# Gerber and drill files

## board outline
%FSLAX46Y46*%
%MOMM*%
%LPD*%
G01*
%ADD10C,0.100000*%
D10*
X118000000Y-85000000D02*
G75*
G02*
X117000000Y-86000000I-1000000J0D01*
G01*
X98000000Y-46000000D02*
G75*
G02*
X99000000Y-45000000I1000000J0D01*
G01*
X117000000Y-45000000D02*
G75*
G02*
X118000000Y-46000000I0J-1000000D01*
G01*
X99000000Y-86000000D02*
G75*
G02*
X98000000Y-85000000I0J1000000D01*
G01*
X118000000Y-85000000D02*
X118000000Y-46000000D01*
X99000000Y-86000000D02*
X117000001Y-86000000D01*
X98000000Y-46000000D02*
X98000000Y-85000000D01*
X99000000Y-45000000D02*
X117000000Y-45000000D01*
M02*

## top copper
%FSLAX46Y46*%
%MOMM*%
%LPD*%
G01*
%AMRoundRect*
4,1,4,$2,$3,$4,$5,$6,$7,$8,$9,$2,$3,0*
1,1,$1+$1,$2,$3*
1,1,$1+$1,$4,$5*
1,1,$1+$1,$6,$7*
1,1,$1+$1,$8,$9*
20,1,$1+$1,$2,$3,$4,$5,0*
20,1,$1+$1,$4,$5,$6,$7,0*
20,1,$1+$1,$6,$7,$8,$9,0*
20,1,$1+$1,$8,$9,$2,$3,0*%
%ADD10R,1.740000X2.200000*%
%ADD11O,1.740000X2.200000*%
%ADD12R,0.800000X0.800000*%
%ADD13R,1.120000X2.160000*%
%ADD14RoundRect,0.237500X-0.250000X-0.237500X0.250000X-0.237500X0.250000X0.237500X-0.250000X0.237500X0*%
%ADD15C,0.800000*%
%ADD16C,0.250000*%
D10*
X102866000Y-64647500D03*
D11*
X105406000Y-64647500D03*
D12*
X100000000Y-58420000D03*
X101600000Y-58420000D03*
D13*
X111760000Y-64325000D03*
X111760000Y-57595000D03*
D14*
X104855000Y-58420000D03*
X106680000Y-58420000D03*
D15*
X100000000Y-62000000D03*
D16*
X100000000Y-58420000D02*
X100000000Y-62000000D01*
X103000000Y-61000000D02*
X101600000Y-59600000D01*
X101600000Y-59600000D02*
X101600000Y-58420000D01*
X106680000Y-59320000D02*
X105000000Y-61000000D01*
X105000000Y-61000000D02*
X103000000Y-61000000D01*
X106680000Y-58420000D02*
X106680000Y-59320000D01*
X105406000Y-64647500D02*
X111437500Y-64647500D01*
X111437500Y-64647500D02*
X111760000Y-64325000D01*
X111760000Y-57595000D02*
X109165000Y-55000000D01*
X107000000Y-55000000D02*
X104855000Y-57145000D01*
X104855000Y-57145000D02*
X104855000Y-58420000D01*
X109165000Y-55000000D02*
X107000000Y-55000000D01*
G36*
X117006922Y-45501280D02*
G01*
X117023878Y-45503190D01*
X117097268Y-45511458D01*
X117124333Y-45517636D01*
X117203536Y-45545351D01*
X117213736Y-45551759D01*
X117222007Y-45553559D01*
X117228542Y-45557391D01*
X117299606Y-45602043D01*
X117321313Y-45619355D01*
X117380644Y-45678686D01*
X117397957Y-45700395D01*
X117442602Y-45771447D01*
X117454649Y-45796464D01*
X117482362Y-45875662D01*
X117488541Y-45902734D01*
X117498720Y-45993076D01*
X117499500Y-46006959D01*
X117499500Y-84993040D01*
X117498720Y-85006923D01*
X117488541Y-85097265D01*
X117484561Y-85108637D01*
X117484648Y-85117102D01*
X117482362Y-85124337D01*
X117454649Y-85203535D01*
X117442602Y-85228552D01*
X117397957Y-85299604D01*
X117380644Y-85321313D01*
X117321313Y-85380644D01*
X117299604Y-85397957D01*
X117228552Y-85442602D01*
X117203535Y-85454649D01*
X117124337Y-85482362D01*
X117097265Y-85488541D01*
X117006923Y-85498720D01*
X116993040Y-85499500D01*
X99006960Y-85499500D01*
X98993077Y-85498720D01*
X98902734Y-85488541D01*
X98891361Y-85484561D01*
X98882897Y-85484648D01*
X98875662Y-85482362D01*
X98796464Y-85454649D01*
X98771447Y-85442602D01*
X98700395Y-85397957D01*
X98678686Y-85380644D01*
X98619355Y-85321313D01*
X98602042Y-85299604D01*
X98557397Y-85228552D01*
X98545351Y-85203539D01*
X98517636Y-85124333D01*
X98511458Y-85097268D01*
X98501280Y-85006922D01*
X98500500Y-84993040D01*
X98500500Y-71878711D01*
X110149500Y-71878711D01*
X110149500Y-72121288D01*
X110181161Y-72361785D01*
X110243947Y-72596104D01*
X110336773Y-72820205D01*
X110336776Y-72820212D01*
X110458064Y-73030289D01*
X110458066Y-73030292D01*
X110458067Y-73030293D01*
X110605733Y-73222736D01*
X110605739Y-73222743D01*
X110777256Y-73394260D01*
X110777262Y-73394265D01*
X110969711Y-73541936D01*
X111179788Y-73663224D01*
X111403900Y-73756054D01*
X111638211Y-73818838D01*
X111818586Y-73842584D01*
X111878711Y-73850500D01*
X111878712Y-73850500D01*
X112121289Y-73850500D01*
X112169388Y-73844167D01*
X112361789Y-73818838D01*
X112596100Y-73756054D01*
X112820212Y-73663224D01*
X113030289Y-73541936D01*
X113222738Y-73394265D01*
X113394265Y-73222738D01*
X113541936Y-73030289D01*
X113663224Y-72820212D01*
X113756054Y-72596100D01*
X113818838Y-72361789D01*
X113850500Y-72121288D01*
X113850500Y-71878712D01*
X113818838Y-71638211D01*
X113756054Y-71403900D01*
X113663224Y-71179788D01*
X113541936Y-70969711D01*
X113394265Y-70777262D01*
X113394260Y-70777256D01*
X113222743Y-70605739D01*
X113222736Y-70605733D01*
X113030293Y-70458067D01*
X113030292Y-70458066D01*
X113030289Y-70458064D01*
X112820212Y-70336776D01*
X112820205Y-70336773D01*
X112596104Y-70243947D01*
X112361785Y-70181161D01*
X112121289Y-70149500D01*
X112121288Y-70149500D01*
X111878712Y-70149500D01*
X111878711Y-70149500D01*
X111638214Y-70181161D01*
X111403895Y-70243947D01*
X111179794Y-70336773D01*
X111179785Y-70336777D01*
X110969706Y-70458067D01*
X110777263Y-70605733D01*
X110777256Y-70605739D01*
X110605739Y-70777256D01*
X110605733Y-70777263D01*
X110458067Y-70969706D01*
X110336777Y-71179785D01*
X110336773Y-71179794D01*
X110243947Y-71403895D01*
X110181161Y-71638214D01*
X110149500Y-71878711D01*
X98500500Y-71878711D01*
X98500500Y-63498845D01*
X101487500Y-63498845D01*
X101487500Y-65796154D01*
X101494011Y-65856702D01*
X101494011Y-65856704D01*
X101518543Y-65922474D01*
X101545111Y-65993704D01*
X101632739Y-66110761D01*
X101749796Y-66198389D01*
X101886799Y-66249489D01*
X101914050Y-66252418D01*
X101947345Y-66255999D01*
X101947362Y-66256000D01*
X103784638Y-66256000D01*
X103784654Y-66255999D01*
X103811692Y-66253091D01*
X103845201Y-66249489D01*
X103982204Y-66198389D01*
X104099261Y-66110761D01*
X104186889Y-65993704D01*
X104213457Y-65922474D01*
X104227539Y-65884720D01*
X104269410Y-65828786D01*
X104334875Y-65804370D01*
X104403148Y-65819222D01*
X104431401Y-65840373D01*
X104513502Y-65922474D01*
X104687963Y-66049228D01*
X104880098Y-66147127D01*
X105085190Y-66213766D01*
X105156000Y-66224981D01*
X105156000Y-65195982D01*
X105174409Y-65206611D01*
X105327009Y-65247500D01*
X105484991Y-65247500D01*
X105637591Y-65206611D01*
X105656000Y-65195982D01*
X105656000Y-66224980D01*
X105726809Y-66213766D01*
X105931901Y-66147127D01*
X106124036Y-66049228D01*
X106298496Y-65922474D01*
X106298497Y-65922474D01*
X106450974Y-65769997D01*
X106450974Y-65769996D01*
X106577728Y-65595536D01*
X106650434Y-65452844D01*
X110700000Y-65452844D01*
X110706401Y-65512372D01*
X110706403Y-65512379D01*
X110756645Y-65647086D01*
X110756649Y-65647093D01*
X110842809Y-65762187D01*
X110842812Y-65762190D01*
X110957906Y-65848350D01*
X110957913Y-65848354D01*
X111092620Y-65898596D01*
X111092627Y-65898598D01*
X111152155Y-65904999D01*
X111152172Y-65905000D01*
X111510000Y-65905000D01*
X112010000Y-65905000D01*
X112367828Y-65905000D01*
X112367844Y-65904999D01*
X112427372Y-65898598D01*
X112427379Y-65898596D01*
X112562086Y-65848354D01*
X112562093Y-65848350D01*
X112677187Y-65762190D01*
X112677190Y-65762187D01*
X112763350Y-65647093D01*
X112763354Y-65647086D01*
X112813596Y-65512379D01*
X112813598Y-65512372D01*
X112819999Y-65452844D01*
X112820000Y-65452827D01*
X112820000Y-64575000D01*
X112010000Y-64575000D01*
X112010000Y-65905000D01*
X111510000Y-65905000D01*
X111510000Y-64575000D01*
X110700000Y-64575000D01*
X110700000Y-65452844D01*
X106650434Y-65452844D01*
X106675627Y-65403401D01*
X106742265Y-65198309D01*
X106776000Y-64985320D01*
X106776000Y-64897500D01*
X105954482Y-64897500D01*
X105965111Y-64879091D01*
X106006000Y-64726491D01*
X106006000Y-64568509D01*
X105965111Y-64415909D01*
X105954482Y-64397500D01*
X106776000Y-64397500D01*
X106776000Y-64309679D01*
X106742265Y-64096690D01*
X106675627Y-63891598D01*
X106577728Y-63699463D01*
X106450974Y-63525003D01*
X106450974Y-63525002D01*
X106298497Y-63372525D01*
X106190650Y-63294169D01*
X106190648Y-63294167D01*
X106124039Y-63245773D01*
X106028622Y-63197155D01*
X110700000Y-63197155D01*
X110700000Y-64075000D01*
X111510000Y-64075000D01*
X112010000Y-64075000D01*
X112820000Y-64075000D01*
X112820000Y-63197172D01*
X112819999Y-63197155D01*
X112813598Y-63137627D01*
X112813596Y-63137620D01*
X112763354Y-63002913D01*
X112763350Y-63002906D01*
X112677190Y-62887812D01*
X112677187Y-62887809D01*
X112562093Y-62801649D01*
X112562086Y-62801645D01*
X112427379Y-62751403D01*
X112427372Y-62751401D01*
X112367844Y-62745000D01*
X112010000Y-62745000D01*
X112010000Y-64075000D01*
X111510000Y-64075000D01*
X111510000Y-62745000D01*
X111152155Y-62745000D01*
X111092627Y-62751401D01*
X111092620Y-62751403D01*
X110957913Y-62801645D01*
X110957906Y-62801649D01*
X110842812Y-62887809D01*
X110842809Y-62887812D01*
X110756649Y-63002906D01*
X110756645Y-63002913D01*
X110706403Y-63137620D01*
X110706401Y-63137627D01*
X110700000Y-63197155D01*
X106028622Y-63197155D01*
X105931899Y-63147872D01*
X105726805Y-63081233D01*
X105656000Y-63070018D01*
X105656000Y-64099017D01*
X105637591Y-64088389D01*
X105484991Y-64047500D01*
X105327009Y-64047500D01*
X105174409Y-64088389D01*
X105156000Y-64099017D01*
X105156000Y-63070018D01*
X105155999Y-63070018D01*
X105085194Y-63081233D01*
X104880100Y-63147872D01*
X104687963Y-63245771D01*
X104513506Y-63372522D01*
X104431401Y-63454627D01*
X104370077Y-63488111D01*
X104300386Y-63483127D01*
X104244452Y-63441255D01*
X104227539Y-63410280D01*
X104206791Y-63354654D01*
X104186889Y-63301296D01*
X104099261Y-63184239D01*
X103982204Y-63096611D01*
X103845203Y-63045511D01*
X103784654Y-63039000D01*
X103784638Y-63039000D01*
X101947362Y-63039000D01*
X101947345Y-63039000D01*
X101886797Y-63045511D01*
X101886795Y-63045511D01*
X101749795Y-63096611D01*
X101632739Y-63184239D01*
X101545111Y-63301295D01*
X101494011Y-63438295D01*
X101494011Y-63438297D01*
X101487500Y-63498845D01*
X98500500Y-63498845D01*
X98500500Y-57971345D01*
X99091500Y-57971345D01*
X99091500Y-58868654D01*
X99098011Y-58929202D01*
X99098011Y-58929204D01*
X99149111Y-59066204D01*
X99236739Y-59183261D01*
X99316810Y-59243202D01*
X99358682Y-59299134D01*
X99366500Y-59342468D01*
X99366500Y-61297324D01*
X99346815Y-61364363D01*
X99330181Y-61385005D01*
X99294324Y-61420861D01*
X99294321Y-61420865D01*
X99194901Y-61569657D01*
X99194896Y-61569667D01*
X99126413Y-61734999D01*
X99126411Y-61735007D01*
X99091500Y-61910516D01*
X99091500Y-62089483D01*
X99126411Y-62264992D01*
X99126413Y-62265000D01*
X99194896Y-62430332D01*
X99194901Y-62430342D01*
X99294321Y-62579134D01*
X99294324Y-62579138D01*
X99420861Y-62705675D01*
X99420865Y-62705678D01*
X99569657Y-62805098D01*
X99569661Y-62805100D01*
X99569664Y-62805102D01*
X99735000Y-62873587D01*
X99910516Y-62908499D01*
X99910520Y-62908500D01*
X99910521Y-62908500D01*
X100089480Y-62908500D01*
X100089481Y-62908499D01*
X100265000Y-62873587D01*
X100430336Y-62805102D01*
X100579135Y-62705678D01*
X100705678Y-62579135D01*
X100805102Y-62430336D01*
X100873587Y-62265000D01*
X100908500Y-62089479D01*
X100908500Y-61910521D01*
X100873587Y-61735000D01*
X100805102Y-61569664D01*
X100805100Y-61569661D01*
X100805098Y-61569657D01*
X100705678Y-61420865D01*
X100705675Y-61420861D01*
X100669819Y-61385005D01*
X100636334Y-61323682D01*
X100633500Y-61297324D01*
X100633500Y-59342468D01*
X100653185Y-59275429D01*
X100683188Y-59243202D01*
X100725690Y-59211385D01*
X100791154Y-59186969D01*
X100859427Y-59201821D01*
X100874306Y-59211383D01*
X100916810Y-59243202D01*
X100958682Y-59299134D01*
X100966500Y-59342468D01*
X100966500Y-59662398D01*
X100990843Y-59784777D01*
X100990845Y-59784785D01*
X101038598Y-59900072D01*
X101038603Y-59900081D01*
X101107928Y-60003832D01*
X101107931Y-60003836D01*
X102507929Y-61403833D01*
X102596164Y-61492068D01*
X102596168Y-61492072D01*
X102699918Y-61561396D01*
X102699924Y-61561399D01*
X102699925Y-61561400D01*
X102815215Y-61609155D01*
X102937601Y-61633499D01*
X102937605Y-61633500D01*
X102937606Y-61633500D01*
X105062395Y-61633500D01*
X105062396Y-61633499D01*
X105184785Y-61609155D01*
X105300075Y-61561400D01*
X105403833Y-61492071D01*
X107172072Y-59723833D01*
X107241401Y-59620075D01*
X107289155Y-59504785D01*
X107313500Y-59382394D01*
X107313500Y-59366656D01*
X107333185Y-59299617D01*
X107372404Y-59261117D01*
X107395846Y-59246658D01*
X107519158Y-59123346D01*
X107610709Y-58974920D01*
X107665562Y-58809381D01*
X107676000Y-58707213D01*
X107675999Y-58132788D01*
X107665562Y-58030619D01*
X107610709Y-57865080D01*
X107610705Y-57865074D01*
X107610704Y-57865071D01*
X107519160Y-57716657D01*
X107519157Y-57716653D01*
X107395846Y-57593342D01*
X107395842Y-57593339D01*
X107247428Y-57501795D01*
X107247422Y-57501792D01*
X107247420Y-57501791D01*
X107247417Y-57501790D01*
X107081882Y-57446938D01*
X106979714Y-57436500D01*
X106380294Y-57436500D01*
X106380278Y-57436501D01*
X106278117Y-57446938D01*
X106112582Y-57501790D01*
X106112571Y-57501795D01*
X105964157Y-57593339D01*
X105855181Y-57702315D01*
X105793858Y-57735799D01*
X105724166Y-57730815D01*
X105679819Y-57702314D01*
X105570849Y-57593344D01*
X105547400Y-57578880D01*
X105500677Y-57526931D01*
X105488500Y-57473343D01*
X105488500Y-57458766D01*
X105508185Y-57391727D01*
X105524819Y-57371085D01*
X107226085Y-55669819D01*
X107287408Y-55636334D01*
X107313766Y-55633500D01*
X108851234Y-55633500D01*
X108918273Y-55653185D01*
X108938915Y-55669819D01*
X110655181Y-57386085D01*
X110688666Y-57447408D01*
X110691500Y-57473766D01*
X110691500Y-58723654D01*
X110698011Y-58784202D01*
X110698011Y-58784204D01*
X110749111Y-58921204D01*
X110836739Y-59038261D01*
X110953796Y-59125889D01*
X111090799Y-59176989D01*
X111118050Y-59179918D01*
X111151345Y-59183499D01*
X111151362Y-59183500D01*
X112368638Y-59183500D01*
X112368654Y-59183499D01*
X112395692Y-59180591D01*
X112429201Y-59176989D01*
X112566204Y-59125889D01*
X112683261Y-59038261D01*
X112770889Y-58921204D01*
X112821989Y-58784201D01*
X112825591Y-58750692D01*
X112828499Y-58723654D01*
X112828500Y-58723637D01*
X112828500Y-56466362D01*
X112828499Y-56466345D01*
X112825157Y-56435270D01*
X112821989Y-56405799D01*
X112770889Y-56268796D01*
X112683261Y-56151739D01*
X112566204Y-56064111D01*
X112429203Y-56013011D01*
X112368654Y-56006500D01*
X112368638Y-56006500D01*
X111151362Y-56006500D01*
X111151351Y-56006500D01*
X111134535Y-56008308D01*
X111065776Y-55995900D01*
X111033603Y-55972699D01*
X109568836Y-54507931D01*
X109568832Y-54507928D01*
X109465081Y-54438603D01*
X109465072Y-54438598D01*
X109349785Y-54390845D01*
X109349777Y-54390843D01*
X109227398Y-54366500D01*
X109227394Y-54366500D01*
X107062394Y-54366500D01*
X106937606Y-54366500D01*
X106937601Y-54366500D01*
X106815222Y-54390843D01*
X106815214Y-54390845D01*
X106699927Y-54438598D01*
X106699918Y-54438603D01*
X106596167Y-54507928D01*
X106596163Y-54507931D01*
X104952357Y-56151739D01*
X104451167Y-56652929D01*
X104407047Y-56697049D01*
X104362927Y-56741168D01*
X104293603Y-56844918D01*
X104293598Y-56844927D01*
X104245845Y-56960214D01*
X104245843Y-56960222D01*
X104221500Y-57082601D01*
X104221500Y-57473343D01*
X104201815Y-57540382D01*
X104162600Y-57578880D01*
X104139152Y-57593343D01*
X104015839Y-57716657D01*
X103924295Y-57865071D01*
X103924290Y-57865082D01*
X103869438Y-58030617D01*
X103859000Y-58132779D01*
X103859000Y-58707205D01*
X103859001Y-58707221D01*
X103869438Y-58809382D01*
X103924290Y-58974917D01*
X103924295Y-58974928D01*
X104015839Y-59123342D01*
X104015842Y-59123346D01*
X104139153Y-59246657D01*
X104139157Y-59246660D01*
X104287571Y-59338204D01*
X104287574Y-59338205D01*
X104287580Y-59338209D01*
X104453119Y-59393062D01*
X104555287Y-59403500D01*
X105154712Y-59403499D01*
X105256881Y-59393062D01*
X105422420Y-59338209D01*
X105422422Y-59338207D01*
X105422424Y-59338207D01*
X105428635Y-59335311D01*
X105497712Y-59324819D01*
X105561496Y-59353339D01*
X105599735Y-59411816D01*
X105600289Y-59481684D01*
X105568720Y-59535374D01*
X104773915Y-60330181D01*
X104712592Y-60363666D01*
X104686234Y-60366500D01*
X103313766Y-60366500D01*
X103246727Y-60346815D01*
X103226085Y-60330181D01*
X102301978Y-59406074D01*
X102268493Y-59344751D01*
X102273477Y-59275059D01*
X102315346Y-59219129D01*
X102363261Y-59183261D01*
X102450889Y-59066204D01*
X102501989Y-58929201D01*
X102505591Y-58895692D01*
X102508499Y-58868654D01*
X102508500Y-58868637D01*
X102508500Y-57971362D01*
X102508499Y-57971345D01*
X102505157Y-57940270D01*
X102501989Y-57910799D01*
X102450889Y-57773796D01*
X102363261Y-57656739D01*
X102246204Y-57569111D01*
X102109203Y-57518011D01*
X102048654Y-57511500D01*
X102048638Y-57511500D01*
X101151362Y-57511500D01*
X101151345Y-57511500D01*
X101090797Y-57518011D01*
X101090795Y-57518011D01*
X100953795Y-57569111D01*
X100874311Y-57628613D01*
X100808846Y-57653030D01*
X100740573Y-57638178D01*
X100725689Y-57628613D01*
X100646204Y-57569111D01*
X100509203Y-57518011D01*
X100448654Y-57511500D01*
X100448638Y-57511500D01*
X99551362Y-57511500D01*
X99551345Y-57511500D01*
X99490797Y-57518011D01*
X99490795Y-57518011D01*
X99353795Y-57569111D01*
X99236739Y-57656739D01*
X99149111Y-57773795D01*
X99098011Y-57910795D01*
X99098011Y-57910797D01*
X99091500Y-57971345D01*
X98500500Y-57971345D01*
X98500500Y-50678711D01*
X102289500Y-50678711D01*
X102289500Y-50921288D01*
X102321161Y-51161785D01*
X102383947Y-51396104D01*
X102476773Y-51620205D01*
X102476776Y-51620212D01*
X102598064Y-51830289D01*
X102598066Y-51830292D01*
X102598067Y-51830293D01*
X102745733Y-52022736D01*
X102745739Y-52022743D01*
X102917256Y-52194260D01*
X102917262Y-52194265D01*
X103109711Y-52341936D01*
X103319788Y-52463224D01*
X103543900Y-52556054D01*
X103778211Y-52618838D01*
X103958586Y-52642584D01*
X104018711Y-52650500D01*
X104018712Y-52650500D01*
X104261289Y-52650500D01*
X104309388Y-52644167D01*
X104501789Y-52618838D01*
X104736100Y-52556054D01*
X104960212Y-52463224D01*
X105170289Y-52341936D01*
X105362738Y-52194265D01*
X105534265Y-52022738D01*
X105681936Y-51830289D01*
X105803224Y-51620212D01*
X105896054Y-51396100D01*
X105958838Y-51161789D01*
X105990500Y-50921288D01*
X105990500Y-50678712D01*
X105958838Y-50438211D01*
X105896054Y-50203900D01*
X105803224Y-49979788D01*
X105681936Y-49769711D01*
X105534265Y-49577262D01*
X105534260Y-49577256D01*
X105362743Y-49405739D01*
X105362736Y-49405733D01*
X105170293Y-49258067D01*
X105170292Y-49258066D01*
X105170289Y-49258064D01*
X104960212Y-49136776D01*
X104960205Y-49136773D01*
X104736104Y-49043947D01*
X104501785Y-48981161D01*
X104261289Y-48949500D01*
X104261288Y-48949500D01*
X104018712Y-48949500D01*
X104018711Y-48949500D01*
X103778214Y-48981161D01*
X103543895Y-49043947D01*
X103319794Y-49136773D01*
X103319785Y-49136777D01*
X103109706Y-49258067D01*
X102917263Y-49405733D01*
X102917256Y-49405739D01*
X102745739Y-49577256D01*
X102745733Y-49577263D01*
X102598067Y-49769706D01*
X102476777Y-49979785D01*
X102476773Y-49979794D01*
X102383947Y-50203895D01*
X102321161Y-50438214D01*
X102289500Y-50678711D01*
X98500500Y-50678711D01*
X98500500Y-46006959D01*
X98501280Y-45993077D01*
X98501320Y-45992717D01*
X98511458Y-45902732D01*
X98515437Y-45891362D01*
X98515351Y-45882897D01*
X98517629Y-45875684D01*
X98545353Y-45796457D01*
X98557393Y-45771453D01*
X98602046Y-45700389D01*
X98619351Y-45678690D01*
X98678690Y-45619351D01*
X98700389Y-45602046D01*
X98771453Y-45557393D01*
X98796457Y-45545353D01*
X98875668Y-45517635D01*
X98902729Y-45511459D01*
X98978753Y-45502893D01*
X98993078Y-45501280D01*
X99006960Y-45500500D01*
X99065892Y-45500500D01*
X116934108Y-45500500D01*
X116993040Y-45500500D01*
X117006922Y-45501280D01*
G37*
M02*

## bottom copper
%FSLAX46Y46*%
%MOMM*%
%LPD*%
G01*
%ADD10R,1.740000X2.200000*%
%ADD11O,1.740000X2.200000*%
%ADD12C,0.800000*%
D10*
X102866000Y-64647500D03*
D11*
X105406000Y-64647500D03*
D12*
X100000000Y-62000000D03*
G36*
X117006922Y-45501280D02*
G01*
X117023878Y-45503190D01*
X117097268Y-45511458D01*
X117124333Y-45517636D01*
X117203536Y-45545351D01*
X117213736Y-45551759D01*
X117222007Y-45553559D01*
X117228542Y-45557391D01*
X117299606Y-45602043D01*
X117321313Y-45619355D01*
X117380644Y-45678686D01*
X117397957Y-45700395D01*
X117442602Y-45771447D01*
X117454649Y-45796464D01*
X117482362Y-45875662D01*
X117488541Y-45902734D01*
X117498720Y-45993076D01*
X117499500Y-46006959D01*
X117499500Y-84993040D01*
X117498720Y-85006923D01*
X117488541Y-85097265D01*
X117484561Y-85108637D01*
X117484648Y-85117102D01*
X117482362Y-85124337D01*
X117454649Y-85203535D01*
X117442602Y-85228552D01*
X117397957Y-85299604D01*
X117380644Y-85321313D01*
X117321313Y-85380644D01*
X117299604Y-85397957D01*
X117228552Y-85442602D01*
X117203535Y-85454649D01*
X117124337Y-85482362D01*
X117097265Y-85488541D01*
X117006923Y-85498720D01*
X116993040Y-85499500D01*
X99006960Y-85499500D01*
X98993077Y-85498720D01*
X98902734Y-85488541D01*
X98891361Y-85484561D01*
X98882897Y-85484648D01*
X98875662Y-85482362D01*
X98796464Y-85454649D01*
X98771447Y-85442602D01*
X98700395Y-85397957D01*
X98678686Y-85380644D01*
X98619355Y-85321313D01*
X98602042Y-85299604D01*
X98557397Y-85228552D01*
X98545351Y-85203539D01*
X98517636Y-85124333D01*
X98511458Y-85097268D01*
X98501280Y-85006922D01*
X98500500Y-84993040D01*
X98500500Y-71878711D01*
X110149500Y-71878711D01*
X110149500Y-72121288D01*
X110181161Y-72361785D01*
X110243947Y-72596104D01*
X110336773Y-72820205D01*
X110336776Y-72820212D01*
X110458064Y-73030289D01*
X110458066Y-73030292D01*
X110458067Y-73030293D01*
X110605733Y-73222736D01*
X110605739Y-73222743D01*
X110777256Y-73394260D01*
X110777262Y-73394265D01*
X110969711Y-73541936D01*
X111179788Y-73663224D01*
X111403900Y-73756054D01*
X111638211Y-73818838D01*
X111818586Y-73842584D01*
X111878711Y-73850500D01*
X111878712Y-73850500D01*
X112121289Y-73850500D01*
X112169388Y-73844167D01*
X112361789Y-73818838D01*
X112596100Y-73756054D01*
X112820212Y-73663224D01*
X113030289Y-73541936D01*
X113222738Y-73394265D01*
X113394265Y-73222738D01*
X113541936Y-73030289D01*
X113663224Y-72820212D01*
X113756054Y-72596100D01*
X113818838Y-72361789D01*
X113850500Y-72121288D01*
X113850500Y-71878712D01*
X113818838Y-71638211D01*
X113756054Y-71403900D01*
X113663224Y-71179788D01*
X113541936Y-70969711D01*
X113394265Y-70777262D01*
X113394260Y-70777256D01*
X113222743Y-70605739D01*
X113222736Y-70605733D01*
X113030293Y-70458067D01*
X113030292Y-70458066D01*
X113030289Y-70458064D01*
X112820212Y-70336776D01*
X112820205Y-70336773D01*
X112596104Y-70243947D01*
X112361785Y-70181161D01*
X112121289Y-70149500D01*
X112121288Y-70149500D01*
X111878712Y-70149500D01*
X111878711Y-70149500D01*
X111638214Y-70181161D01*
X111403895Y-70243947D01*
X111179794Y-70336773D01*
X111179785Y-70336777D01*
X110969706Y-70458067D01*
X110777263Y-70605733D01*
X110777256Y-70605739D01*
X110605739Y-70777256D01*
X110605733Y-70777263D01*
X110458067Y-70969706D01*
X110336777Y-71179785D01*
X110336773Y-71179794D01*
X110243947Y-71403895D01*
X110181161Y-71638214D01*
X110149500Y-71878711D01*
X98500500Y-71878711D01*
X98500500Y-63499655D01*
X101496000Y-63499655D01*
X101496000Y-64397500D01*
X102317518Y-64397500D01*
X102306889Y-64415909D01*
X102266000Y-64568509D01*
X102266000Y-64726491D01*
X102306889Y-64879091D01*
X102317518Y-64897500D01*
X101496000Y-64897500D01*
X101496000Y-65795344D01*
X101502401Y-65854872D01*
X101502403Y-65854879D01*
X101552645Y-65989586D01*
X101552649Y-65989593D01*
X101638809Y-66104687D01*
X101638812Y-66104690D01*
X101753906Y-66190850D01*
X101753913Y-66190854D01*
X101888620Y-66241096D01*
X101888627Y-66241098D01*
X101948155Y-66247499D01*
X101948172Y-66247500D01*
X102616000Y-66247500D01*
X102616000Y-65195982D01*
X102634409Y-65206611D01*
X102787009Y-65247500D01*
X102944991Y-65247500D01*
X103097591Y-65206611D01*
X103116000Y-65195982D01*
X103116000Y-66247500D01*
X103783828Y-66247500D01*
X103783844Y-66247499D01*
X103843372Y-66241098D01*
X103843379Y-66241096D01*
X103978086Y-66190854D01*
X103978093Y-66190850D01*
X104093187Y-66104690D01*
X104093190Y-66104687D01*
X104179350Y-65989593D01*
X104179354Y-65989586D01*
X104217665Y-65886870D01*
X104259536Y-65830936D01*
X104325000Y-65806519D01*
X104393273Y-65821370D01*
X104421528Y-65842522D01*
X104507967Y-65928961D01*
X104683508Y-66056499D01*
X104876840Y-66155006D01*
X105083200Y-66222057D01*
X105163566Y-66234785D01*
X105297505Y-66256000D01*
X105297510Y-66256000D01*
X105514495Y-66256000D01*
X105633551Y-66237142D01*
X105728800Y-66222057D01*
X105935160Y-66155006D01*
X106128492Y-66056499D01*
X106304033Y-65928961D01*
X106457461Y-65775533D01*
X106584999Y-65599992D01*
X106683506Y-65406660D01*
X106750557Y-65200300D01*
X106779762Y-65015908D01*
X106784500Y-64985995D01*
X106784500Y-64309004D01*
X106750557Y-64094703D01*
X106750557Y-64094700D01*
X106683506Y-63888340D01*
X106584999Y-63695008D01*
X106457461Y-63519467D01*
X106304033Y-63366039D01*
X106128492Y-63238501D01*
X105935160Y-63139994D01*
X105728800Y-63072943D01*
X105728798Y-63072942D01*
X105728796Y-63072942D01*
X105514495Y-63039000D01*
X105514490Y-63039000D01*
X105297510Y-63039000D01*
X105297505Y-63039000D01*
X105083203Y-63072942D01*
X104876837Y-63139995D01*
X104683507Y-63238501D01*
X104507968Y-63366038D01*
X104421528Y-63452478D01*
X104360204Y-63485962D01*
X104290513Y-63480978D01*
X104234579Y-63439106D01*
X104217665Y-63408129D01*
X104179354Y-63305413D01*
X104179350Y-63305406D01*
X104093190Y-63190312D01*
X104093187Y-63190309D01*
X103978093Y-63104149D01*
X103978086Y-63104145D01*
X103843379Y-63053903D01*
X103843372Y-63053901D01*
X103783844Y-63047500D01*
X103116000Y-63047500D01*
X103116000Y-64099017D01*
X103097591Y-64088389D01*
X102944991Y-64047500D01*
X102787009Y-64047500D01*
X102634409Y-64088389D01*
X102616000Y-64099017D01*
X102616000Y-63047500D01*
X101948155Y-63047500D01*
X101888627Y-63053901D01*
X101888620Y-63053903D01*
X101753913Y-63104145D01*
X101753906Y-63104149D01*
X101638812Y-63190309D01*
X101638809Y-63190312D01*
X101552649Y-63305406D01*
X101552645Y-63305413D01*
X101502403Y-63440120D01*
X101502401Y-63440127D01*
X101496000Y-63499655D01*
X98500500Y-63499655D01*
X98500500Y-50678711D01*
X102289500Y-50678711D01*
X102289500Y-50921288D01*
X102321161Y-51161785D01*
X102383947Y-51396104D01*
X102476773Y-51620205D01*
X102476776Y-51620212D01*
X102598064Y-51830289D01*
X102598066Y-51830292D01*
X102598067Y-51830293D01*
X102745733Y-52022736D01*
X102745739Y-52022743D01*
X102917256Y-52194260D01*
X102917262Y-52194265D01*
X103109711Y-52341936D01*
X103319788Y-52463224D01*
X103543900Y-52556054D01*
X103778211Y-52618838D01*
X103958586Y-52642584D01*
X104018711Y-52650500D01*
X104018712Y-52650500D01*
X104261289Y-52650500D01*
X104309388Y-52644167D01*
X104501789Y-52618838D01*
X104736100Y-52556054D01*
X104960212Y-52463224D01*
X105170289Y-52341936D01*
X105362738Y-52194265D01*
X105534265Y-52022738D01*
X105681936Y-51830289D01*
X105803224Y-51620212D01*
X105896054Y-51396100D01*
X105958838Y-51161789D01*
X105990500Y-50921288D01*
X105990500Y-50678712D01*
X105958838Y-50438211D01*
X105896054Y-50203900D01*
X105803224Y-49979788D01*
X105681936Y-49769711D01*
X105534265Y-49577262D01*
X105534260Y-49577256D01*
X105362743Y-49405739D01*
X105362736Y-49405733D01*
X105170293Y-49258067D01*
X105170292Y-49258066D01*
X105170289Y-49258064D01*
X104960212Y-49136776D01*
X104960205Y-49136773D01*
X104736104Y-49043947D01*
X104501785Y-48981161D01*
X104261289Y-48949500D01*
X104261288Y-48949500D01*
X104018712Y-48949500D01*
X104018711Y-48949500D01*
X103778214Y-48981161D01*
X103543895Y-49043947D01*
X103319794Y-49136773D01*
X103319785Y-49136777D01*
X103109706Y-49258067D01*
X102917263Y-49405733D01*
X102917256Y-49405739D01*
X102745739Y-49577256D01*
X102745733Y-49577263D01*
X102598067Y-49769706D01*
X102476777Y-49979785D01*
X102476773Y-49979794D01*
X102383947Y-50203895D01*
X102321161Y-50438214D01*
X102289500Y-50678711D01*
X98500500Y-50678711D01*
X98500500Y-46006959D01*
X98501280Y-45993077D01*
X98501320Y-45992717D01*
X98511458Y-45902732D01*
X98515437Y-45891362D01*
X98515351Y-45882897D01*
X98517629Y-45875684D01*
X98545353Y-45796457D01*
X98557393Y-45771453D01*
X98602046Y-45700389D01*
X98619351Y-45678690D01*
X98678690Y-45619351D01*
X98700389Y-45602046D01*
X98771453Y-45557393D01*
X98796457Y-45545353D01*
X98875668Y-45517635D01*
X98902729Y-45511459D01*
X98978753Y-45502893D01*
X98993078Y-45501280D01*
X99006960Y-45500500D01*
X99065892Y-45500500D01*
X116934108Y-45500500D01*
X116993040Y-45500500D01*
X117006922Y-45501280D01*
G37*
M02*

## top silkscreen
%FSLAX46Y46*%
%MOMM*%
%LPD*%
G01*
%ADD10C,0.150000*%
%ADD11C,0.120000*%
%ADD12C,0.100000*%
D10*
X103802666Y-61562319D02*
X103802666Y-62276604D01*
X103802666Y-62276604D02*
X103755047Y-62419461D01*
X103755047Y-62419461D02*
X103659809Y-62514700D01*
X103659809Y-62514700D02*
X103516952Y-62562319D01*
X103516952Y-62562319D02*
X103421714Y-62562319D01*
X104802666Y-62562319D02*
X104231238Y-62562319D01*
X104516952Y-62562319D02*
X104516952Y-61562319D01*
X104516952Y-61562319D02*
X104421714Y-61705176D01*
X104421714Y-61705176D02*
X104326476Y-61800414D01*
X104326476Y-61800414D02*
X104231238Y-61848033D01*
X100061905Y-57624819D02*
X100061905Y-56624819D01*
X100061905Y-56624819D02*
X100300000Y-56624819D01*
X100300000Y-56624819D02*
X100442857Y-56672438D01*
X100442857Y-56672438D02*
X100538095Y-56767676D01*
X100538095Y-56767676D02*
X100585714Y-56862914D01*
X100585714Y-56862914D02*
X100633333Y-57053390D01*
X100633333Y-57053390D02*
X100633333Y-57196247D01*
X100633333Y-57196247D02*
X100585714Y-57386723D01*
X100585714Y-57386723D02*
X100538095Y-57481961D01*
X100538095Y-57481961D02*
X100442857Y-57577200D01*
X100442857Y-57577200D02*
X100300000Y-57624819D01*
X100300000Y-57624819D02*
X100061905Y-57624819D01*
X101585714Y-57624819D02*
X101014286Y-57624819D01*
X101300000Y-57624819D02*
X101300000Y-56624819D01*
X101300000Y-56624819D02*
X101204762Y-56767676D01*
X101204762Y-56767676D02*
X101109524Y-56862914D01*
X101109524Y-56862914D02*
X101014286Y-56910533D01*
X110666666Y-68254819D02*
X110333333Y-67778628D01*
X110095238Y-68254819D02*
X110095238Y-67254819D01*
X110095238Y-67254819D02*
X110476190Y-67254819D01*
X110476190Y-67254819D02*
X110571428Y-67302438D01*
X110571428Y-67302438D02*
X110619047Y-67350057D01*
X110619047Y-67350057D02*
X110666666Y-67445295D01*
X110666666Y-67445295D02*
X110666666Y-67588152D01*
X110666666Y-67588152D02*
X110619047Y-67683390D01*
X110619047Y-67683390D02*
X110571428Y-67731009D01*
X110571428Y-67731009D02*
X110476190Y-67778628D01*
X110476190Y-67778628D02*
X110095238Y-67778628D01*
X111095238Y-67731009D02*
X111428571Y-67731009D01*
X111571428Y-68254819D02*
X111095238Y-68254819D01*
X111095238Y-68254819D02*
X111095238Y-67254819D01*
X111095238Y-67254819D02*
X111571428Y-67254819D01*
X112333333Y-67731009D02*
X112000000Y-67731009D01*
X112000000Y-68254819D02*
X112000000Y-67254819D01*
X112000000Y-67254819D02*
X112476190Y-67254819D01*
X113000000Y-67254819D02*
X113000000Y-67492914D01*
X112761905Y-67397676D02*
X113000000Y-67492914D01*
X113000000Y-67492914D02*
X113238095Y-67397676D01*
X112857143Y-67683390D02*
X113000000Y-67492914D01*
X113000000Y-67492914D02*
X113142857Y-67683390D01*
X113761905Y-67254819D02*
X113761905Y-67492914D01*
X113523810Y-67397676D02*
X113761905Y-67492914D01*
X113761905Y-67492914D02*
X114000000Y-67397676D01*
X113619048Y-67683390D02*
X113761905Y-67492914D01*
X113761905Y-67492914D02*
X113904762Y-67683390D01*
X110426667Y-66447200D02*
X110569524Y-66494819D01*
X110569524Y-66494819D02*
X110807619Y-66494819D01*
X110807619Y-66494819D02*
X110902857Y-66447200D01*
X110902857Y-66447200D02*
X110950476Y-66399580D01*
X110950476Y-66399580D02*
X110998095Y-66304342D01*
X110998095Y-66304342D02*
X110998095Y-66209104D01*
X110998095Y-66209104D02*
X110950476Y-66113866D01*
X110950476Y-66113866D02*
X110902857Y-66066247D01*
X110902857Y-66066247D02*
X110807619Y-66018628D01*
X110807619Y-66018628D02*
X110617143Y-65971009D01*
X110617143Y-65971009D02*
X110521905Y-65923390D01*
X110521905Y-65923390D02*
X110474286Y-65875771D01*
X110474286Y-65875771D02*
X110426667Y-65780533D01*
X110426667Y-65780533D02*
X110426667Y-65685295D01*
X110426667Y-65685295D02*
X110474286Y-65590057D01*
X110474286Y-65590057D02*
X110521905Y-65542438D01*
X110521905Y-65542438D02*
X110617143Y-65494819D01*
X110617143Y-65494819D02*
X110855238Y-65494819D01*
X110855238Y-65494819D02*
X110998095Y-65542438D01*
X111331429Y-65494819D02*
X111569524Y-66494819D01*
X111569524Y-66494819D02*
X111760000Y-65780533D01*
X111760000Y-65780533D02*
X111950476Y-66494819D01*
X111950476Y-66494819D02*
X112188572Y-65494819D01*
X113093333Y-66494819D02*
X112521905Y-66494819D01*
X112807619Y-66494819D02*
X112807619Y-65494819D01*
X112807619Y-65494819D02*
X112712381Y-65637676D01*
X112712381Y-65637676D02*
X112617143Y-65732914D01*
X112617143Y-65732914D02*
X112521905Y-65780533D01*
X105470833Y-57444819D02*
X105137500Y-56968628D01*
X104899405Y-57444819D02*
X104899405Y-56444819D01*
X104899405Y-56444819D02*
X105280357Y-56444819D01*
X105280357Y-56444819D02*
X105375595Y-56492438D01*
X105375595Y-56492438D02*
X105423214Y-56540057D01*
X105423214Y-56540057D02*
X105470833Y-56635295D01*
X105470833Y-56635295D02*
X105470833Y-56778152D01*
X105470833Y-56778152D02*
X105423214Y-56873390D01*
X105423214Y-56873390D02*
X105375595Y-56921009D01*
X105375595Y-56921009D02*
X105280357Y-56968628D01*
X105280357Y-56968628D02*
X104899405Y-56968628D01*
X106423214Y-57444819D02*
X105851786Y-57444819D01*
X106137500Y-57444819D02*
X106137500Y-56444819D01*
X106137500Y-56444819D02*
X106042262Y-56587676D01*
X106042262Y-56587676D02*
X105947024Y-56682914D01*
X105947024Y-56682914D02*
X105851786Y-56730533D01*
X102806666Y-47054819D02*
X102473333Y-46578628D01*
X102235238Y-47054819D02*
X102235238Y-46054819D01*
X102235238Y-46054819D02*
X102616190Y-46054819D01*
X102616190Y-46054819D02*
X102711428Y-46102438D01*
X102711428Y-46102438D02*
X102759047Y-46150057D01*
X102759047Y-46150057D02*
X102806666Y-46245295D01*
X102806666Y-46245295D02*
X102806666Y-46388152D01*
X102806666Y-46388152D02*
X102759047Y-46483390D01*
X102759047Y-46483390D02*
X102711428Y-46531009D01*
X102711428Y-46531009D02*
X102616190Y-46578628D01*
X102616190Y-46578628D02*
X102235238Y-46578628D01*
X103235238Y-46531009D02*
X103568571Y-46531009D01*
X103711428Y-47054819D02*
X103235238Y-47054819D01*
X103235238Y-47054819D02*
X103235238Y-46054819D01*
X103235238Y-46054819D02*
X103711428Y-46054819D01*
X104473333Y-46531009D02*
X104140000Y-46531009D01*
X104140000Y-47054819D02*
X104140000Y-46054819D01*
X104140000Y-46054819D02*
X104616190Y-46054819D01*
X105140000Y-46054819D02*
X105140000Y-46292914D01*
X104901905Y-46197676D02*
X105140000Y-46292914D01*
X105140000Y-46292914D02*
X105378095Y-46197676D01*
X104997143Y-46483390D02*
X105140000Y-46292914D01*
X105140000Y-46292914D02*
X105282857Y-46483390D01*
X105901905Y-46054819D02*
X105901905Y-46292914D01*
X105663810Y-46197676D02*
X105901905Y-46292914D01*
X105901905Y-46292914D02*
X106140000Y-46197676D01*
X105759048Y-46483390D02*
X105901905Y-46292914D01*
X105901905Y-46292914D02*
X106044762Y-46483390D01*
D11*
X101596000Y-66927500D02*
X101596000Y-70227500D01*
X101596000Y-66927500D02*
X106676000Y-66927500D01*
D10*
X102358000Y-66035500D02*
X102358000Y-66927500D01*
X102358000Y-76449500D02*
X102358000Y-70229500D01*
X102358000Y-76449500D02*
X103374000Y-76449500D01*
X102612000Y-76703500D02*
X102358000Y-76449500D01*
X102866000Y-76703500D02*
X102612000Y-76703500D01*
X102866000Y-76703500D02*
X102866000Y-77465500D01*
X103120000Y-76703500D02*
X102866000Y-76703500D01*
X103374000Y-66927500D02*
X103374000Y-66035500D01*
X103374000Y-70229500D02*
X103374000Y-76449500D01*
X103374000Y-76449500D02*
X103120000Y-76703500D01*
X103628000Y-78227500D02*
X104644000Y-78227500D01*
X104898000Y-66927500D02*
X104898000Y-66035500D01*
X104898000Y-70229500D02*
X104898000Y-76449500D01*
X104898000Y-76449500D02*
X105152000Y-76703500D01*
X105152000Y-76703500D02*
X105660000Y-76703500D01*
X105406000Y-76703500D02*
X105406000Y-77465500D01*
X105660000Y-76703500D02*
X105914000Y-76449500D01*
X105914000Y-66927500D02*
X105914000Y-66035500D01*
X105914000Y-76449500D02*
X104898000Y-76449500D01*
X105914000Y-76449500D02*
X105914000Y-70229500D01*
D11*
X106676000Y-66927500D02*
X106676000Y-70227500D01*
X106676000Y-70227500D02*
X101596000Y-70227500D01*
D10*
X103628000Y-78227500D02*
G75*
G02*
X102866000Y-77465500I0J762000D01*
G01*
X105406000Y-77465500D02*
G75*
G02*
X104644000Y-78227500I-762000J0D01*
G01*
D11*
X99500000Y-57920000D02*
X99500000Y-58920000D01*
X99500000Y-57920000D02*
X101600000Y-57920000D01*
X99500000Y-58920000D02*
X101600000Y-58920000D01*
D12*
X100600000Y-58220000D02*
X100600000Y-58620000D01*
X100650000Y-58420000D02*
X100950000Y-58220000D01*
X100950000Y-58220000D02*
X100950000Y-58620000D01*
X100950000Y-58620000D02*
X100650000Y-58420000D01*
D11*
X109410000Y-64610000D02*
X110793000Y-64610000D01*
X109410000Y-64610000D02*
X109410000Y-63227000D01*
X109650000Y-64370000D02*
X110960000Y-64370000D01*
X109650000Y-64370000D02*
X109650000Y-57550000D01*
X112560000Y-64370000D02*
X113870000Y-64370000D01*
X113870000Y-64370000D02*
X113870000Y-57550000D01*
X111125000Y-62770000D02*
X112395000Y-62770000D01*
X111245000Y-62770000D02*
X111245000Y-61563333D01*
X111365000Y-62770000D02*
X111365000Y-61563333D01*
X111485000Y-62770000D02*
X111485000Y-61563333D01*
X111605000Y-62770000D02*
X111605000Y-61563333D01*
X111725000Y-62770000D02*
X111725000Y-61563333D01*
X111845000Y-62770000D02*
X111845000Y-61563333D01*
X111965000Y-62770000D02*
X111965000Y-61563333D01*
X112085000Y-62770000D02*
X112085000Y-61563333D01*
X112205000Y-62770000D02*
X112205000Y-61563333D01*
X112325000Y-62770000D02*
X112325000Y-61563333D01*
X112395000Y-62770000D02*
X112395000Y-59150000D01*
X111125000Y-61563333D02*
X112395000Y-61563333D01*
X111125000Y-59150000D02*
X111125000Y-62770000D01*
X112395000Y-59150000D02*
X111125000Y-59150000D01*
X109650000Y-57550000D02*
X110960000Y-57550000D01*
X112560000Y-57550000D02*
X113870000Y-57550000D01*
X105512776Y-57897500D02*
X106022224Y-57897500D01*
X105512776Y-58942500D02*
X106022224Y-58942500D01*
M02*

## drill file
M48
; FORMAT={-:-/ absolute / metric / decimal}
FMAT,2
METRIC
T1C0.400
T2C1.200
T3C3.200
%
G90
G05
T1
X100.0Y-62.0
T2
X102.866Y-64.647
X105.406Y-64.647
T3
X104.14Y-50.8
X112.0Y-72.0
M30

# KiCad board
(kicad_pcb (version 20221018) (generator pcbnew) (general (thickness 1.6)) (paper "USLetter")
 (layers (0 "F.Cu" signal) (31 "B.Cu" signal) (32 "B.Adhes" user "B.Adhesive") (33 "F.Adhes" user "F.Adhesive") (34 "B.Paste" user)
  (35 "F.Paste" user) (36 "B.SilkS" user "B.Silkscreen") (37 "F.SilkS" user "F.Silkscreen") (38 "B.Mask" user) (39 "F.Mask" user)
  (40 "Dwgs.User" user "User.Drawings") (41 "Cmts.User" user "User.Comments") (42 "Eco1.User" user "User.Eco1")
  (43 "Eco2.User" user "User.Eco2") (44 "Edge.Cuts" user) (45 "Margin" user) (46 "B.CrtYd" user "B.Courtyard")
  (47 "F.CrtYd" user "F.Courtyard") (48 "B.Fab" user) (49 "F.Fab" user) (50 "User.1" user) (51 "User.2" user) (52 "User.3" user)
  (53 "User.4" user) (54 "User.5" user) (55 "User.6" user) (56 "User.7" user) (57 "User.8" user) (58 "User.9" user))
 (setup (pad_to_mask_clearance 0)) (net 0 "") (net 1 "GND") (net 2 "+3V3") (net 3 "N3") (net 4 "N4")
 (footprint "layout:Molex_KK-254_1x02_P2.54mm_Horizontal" (layer "F.Cu") (at 102.866 64.6475)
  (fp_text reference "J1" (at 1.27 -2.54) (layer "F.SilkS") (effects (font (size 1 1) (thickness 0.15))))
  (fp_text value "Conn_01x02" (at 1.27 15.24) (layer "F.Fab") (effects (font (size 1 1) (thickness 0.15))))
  (fp_line (start -1.27 2.28) (end -1.27 5.58) (stroke (width 0.12) (type solid)) (layer "F.SilkS"))
  (fp_line (start -1.27 2.28) (end 3.81 2.28) (stroke (width 0.12) (type solid)) (layer "F.SilkS"))
  (fp_line (start -0.508 1.388) (end -0.508 2.28) (stroke (width 0.15) (type solid)) (layer "F.SilkS"))
  (fp_line (start -0.508 11.802) (end -0.508 5.582) (stroke (width 0.15) (type solid)) (layer "F.SilkS"))
  (fp_line (start -0.508 11.802) (end 0.508 11.802) (stroke (width 0.15) (type solid)) (layer "F.SilkS"))
  (fp_line (start -0.254 12.056) (end -0.508 11.802) (stroke (width 0.15) (type solid)) (layer "F.SilkS"))
  (fp_line (start 0 12.056) (end -0.254 12.056) (stroke (width 0.15) (type solid)) (layer "F.SilkS"))
  (fp_line (start 0 12.056) (end 0 12.818) (stroke (width 0.15) (type solid)) (layer "F.SilkS"))
  (fp_line (start 0.254 12.056) (end 0 12.056) (stroke (width 0.15) (type solid)) (layer "F.SilkS"))
  (fp_line (start 0.508 2.28) (end 0.508 1.388) (stroke (width 0.15) (type solid)) (layer "F.SilkS"))
  (fp_line (start 0.508 5.582) (end 0.508 11.802) (stroke (width 0.15) (type solid)) (layer "F.SilkS"))
  (fp_line (start 0.508 11.802) (end 0.254 12.056) (stroke (width 0.15) (type solid)) (layer "F.SilkS"))
  (fp_line (start 0.762 13.58) (end 1.778 13.58) (stroke (width 0.15) (type solid)) (layer "F.SilkS"))
  (fp_line (start 2.032 2.28) (end 2.032 1.388) (stroke (width 0.15) (type solid)) (layer "F.SilkS"))
  (fp_line (start 2.032 5.582) (end 2.032 11.802) (stroke (width 0.15) (type solid)) (layer "F.SilkS"))
  (fp_line (start 2.032 11.802) (end 2.286 12.056) (stroke (width 0.15) (type solid)) (layer "F.SilkS"))
  (fp_line (start 2.286 12.056) (end 2.794 12.056) (stroke (width 0.15) (type solid)) (layer "F.SilkS"))
  (fp_line (start 2.54 12.056) (end 2.54 12.818) (stroke (width 0.15) (type solid)) (layer "F.SilkS"))
  (fp_line (start 2.794 12.056) (end 3.048 11.802) (stroke (width 0.15) (type solid)) (layer "F.SilkS"))
  (fp_line (start 3.048 2.28) (end 3.048 1.388) (stroke (width 0.15) (type solid)) (layer "F.SilkS"))
  (fp_line (start 3.048 11.802) (end 2.032 11.802) (stroke (width 0.15) (type solid)) (layer "F.SilkS"))
  (fp_line (start 3.048 11.802) (end 3.048 5.582) (stroke (width 0.15) (type solid)) (layer "F.SilkS"))
  (fp_line (start 3.81 2.28) (end 3.81 5.58) (stroke (width 0.12) (type solid)) (layer "F.SilkS"))
  (fp_line (start 3.81 5.58) (end -1.27 5.58) (stroke (width 0.12) (type solid)) (layer "F.SilkS"))
  (fp_arc (start 0.762 13.58) (mid 0.223185 13.356815) (end 0 12.818) (stroke (width 0.15) (type solid)) (layer "F.SilkS"))
  (fp_arc (start 2.54 12.818) (mid 2.316815 13.356815) (end 1.778 13.58) (stroke (width 0.15) (type solid)) (layer "F.SilkS"))
  (pad "1" thru_hole rect (at 0 0) (size 1.74 2.2) (drill 1.2) (layers "*.Cu" "*.Mask") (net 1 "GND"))
  (pad "2" thru_hole oval (at 2.54 0) (size 1.74 2.2) (drill 1.2) (layers "*.Cu" "*.Mask") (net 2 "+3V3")))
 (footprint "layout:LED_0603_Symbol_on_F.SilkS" (layer "F.Cu") (at 100.8 58.42)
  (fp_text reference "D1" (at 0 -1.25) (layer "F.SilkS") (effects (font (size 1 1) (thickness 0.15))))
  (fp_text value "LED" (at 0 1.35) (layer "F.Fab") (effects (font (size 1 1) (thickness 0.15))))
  (fp_line (start -1.3 -0.5) (end -1.3 0.5) (stroke (width 0.12) (type solid)) (layer "F.SilkS"))
  (fp_line (start -1.3 -0.5) (end 0.8 -0.5) (stroke (width 0.12) (type solid)) (layer "F.SilkS"))
  (fp_line (start -1.3 0.5) (end 0.8 0.5) (stroke (width 0.12) (type solid)) (layer "F.SilkS"))
  (fp_line (start -0.2 -0.2) (end -0.2 0.2) (stroke (width 0.1) (type solid)) (layer "F.SilkS"))
  (fp_line (start -0.15 0) (end 0.15 -0.2) (stroke (width 0.1) (type solid)) (layer "F.SilkS"))
  (fp_line (start 0.15 -0.2) (end 0.15 0.2) (stroke (width 0.1) (type solid)) (layer "F.SilkS"))
  (fp_line (start 0.15 0.2) (end -0.15 0) (stroke (width 0.1) (type solid)) (layer "F.SilkS"))
  (pad "1" smd rect (at -0.8 0 180) (size 0.8 0.8) (layers "F.Cu" "F.Paste" "F.Mask") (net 1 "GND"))
  (pad "2" smd rect (at 0.8 0 180) (size 0.8 0.8) (layers "F.Cu" "F.Paste" "F.Mask") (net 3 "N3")))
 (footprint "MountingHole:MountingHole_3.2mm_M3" (layer "F.Cu") (at 112 72)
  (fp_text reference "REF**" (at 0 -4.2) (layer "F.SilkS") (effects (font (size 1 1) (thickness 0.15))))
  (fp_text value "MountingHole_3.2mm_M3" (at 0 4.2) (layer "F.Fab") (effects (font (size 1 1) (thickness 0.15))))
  (pad "" np_thru_hole circle (at 0 0) (size 3.2 3.2) (drill 3.2) (layers "F&B.Cu" "*.Mask")))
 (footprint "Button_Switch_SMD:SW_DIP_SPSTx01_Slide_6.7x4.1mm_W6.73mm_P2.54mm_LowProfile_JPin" (layer "F.Cu") (at 111.76 60.96 90)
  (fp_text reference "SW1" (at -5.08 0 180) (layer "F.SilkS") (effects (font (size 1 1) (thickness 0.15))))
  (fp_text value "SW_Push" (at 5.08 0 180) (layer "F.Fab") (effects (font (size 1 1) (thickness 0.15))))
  (fp_line (start -3.65 -2.35) (end -3.65 -0.967) (stroke (width 0.12) (type solid)) (layer "F.SilkS"))
  (fp_line (start -3.65 -2.35) (end -2.267 -2.35) (stroke (width 0.12) (type solid)) (layer "F.SilkS"))
  (fp_line (start -3.41 -2.11) (end -3.41 -0.8) (stroke (width 0.12) (type solid)) (layer "F.SilkS"))
  (fp_line (start -3.41 -2.11) (end 3.41 -2.11) (stroke (width 0.12) (type solid)) (layer "F.SilkS"))
  (fp_line (start -3.41 0.8) (end -3.41 2.11) (stroke (width 0.12) (type solid)) (layer "F.SilkS"))
  (fp_line (start -3.41 2.11) (end 3.41 2.11) (stroke (width 0.12) (type solid)) (layer "F.SilkS"))
  (fp_line (start -1.81 -0.635) (end -1.81 0.635) (stroke (width 0.12) (type solid)) (layer "F.SilkS"))
  (fp_line (start -1.81 -0.515) (end -0.603333 -0.515) (stroke (width 0.12) (type solid)) (layer "F.SilkS"))
  (fp_line (start -1.81 -0.395) (end -0.603333 -0.395) (stroke (width 0.12) (type solid)) (layer "F.SilkS"))
  (fp_line (start -1.81 -0.275) (end -0.603333 -0.275) (stroke (width 0.12) (type solid)) (layer "F.SilkS"))
  (fp_line (start -1.81 -0.155) (end -0.603333 -0.155) (stroke (width 0.12) (type solid)) (layer "F.SilkS"))
  (fp_line (start -1.81 -0.035) (end -0.603333 -0.035) (stroke (width 0.12) (type solid)) (layer "F.SilkS"))
  (fp_line (start -1.81 0.085) (end -0.603333 0.085) (stroke (width 0.12) (type solid)) (layer "F.SilkS"))
  (fp_line (start -1.81 0.205) (end -0.603333 0.205) (stroke (width 0.12) (type solid)) (layer "F.SilkS"))
  (fp_line (start -1.81 0.325) (end -0.603333 0.325) (stroke (width 0.12) (type solid)) (layer "F.SilkS"))
  (fp_line (start -1.81 0.445) (end -0.603333 0.445) (stroke (width 0.12) (type solid)) (layer "F.SilkS"))
  (fp_line (start -1.81 0.565) (end -0.603333 0.565) (stroke (width 0.12) (type solid)) (layer "F.SilkS"))
  (fp_line (start -1.81 0.635) (end 1.81 0.635) (stroke (width 0.12) (type solid)) (layer "F.SilkS"))
  (fp_line (start -0.603333 -0.635) (end -0.603333 0.635) (stroke (width 0.12) (type solid)) (layer "F.SilkS"))
  (fp_line (start 1.81 -0.635) (end -1.81 -0.635) (stroke (width 0.12) (type solid)) (layer "F.SilkS"))
  (fp_line (start 1.81 0.635) (end 1.81 -0.635) (stroke (width 0.12) (type solid)) (layer "F.SilkS"))
  (fp_line (start 3.41 -2.11) (end 3.41 -0.8) (stroke (width 0.12) (type solid)) (layer "F.SilkS"))
  (fp_line (start 3.41 0.8) (end 3.41 2.11) (stroke (width 0.12) (type solid)) (layer "F.SilkS"))
  (pad "1" smd rect (at -3.365 0 90) (size 2.16 1.12) (layers "F.Cu" "F.Paste" "F.Mask") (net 2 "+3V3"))
  (pad "2" smd rect (at 3.365 0 90) (size 2.16 1.12) (layers "F.Cu" "F.Paste" "F.Mask") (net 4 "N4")))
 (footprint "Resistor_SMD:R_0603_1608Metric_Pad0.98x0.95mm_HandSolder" (layer "F.Cu") (at 105.7675 58.42)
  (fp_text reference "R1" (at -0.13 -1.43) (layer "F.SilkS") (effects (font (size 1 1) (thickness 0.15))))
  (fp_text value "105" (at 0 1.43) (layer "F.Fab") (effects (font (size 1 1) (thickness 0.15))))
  (fp_line (start -0.254724 -0.5225) (end 0.254724 -0.5225) (stroke (width 0.12) (type solid)) (layer "F.SilkS"))
  (fp_line (start -0.254724 0.5225) (end 0.254724 0.5225) (stroke (width 0.12) (type solid)) (layer "F.SilkS"))
  (pad "1" smd roundrect (at -0.9125 0) (size 0.975 0.95) (layers "F.Cu" "F.Paste" "F.Mask") (roundrect_rratio 0.25) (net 4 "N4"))
  (pad "2" smd roundrect (at 0.9125 0) (size 0.975 0.95) (layers "F.Cu" "F.Paste" "F.Mask") (roundrect_rratio 0.25) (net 3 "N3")))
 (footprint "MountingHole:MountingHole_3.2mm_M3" (layer "F.Cu") (at 104.14 50.8)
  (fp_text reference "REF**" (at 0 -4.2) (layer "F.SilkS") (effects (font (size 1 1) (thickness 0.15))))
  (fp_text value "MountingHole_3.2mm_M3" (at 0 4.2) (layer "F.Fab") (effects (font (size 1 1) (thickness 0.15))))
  (pad "" np_thru_hole circle (at 0 0) (size 3.2 3.2) (drill 3.2) (layers "F&B.Cu" "*.Mask")))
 (gr_arc (start 118 85) (mid 117.707107 85.707107) (end 117 86) (stroke (width 0.1) (type default)) (layer "Edge.Cuts"))
 (gr_arc (start 98 46) (mid 98.292893 45.292893) (end 99 45) (stroke (width 0.1) (type default)) (layer "Edge.Cuts"))
 (gr_arc (start 117 45) (mid 117.707107 45.292893) (end 118 46) (stroke (width 0.1) (type default)) (layer "Edge.Cuts"))
 (gr_arc (start 99 86) (mid 98.292893 85.707107) (end 98 85) (stroke (width 0.1) (type default)) (layer "Edge.Cuts"))
 (gr_line (start 118 85) (end 118 46) (stroke (width 0.1) (type default)) (layer "Edge.Cuts"))
 (gr_line (start 99 86) (end 117.000001 86) (stroke (width 0.1) (type default)) (layer "Edge.Cuts"))
 (gr_line (start 98 46) (end 98 85) (stroke (width 0.1) (type default)) (layer "Edge.Cuts"))
 (gr_line (start 99 45) (end 117 45) (stroke (width 0.1) (type default)) (layer "Edge.Cuts"))
 (segment (start 100 58.42) (end 100 62) (width 0.25) (layer "F.Cu") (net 1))
 (via (at 100 62) (size 0.8) (drill 0.4) (layers "F.Cu" "B.Cu") (free) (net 1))
 (segment (start 103 61) (end 101.6 59.6) (width 0.25) (layer "F.Cu") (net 3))
 (segment (start 101.6 59.6) (end 101.6 58.42) (width 0.25) (layer "F.Cu") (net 3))
 (segment (start 106.68 59.32) (end 105 61) (width 0.25) (layer "F.Cu") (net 3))
 (segment (start 105 61) (end 103 61) (width 0.25) (layer "F.Cu") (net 3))
 (segment (start 106.68 58.42) (end 106.68 59.32) (width 0.25) (layer "F.Cu") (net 3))
 (segment (start 105.406 64.6475) (end 111.4375 64.6475) (width 0.25) (layer "F.Cu") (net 2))
 (segment (start 111.4375 64.6475) (end 111.76 64.325) (width 0.25) (layer "F.Cu") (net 2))
 (segment (start 111.76 57.595) (end 109.165 55) (width 0.25) (layer "F.Cu") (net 4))
 (segment (start 107 55) (end 104.855 57.145) (width 0.25) (layer "F.Cu") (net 4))
 (segment (start 104.855 57.145) (end 104.855 58.42) (width 0.25) (layer "F.Cu") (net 4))
 (segment (start 109.165 55) (end 107 55) (width 0.25) (layer "F.Cu") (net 4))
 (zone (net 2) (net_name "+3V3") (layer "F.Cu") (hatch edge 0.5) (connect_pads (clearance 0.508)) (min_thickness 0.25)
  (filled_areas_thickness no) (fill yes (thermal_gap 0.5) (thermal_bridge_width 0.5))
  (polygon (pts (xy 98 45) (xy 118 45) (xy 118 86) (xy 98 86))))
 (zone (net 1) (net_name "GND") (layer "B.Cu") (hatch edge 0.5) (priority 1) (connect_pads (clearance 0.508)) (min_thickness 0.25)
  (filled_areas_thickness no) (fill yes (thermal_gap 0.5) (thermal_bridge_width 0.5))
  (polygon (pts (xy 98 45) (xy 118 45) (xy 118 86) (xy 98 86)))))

